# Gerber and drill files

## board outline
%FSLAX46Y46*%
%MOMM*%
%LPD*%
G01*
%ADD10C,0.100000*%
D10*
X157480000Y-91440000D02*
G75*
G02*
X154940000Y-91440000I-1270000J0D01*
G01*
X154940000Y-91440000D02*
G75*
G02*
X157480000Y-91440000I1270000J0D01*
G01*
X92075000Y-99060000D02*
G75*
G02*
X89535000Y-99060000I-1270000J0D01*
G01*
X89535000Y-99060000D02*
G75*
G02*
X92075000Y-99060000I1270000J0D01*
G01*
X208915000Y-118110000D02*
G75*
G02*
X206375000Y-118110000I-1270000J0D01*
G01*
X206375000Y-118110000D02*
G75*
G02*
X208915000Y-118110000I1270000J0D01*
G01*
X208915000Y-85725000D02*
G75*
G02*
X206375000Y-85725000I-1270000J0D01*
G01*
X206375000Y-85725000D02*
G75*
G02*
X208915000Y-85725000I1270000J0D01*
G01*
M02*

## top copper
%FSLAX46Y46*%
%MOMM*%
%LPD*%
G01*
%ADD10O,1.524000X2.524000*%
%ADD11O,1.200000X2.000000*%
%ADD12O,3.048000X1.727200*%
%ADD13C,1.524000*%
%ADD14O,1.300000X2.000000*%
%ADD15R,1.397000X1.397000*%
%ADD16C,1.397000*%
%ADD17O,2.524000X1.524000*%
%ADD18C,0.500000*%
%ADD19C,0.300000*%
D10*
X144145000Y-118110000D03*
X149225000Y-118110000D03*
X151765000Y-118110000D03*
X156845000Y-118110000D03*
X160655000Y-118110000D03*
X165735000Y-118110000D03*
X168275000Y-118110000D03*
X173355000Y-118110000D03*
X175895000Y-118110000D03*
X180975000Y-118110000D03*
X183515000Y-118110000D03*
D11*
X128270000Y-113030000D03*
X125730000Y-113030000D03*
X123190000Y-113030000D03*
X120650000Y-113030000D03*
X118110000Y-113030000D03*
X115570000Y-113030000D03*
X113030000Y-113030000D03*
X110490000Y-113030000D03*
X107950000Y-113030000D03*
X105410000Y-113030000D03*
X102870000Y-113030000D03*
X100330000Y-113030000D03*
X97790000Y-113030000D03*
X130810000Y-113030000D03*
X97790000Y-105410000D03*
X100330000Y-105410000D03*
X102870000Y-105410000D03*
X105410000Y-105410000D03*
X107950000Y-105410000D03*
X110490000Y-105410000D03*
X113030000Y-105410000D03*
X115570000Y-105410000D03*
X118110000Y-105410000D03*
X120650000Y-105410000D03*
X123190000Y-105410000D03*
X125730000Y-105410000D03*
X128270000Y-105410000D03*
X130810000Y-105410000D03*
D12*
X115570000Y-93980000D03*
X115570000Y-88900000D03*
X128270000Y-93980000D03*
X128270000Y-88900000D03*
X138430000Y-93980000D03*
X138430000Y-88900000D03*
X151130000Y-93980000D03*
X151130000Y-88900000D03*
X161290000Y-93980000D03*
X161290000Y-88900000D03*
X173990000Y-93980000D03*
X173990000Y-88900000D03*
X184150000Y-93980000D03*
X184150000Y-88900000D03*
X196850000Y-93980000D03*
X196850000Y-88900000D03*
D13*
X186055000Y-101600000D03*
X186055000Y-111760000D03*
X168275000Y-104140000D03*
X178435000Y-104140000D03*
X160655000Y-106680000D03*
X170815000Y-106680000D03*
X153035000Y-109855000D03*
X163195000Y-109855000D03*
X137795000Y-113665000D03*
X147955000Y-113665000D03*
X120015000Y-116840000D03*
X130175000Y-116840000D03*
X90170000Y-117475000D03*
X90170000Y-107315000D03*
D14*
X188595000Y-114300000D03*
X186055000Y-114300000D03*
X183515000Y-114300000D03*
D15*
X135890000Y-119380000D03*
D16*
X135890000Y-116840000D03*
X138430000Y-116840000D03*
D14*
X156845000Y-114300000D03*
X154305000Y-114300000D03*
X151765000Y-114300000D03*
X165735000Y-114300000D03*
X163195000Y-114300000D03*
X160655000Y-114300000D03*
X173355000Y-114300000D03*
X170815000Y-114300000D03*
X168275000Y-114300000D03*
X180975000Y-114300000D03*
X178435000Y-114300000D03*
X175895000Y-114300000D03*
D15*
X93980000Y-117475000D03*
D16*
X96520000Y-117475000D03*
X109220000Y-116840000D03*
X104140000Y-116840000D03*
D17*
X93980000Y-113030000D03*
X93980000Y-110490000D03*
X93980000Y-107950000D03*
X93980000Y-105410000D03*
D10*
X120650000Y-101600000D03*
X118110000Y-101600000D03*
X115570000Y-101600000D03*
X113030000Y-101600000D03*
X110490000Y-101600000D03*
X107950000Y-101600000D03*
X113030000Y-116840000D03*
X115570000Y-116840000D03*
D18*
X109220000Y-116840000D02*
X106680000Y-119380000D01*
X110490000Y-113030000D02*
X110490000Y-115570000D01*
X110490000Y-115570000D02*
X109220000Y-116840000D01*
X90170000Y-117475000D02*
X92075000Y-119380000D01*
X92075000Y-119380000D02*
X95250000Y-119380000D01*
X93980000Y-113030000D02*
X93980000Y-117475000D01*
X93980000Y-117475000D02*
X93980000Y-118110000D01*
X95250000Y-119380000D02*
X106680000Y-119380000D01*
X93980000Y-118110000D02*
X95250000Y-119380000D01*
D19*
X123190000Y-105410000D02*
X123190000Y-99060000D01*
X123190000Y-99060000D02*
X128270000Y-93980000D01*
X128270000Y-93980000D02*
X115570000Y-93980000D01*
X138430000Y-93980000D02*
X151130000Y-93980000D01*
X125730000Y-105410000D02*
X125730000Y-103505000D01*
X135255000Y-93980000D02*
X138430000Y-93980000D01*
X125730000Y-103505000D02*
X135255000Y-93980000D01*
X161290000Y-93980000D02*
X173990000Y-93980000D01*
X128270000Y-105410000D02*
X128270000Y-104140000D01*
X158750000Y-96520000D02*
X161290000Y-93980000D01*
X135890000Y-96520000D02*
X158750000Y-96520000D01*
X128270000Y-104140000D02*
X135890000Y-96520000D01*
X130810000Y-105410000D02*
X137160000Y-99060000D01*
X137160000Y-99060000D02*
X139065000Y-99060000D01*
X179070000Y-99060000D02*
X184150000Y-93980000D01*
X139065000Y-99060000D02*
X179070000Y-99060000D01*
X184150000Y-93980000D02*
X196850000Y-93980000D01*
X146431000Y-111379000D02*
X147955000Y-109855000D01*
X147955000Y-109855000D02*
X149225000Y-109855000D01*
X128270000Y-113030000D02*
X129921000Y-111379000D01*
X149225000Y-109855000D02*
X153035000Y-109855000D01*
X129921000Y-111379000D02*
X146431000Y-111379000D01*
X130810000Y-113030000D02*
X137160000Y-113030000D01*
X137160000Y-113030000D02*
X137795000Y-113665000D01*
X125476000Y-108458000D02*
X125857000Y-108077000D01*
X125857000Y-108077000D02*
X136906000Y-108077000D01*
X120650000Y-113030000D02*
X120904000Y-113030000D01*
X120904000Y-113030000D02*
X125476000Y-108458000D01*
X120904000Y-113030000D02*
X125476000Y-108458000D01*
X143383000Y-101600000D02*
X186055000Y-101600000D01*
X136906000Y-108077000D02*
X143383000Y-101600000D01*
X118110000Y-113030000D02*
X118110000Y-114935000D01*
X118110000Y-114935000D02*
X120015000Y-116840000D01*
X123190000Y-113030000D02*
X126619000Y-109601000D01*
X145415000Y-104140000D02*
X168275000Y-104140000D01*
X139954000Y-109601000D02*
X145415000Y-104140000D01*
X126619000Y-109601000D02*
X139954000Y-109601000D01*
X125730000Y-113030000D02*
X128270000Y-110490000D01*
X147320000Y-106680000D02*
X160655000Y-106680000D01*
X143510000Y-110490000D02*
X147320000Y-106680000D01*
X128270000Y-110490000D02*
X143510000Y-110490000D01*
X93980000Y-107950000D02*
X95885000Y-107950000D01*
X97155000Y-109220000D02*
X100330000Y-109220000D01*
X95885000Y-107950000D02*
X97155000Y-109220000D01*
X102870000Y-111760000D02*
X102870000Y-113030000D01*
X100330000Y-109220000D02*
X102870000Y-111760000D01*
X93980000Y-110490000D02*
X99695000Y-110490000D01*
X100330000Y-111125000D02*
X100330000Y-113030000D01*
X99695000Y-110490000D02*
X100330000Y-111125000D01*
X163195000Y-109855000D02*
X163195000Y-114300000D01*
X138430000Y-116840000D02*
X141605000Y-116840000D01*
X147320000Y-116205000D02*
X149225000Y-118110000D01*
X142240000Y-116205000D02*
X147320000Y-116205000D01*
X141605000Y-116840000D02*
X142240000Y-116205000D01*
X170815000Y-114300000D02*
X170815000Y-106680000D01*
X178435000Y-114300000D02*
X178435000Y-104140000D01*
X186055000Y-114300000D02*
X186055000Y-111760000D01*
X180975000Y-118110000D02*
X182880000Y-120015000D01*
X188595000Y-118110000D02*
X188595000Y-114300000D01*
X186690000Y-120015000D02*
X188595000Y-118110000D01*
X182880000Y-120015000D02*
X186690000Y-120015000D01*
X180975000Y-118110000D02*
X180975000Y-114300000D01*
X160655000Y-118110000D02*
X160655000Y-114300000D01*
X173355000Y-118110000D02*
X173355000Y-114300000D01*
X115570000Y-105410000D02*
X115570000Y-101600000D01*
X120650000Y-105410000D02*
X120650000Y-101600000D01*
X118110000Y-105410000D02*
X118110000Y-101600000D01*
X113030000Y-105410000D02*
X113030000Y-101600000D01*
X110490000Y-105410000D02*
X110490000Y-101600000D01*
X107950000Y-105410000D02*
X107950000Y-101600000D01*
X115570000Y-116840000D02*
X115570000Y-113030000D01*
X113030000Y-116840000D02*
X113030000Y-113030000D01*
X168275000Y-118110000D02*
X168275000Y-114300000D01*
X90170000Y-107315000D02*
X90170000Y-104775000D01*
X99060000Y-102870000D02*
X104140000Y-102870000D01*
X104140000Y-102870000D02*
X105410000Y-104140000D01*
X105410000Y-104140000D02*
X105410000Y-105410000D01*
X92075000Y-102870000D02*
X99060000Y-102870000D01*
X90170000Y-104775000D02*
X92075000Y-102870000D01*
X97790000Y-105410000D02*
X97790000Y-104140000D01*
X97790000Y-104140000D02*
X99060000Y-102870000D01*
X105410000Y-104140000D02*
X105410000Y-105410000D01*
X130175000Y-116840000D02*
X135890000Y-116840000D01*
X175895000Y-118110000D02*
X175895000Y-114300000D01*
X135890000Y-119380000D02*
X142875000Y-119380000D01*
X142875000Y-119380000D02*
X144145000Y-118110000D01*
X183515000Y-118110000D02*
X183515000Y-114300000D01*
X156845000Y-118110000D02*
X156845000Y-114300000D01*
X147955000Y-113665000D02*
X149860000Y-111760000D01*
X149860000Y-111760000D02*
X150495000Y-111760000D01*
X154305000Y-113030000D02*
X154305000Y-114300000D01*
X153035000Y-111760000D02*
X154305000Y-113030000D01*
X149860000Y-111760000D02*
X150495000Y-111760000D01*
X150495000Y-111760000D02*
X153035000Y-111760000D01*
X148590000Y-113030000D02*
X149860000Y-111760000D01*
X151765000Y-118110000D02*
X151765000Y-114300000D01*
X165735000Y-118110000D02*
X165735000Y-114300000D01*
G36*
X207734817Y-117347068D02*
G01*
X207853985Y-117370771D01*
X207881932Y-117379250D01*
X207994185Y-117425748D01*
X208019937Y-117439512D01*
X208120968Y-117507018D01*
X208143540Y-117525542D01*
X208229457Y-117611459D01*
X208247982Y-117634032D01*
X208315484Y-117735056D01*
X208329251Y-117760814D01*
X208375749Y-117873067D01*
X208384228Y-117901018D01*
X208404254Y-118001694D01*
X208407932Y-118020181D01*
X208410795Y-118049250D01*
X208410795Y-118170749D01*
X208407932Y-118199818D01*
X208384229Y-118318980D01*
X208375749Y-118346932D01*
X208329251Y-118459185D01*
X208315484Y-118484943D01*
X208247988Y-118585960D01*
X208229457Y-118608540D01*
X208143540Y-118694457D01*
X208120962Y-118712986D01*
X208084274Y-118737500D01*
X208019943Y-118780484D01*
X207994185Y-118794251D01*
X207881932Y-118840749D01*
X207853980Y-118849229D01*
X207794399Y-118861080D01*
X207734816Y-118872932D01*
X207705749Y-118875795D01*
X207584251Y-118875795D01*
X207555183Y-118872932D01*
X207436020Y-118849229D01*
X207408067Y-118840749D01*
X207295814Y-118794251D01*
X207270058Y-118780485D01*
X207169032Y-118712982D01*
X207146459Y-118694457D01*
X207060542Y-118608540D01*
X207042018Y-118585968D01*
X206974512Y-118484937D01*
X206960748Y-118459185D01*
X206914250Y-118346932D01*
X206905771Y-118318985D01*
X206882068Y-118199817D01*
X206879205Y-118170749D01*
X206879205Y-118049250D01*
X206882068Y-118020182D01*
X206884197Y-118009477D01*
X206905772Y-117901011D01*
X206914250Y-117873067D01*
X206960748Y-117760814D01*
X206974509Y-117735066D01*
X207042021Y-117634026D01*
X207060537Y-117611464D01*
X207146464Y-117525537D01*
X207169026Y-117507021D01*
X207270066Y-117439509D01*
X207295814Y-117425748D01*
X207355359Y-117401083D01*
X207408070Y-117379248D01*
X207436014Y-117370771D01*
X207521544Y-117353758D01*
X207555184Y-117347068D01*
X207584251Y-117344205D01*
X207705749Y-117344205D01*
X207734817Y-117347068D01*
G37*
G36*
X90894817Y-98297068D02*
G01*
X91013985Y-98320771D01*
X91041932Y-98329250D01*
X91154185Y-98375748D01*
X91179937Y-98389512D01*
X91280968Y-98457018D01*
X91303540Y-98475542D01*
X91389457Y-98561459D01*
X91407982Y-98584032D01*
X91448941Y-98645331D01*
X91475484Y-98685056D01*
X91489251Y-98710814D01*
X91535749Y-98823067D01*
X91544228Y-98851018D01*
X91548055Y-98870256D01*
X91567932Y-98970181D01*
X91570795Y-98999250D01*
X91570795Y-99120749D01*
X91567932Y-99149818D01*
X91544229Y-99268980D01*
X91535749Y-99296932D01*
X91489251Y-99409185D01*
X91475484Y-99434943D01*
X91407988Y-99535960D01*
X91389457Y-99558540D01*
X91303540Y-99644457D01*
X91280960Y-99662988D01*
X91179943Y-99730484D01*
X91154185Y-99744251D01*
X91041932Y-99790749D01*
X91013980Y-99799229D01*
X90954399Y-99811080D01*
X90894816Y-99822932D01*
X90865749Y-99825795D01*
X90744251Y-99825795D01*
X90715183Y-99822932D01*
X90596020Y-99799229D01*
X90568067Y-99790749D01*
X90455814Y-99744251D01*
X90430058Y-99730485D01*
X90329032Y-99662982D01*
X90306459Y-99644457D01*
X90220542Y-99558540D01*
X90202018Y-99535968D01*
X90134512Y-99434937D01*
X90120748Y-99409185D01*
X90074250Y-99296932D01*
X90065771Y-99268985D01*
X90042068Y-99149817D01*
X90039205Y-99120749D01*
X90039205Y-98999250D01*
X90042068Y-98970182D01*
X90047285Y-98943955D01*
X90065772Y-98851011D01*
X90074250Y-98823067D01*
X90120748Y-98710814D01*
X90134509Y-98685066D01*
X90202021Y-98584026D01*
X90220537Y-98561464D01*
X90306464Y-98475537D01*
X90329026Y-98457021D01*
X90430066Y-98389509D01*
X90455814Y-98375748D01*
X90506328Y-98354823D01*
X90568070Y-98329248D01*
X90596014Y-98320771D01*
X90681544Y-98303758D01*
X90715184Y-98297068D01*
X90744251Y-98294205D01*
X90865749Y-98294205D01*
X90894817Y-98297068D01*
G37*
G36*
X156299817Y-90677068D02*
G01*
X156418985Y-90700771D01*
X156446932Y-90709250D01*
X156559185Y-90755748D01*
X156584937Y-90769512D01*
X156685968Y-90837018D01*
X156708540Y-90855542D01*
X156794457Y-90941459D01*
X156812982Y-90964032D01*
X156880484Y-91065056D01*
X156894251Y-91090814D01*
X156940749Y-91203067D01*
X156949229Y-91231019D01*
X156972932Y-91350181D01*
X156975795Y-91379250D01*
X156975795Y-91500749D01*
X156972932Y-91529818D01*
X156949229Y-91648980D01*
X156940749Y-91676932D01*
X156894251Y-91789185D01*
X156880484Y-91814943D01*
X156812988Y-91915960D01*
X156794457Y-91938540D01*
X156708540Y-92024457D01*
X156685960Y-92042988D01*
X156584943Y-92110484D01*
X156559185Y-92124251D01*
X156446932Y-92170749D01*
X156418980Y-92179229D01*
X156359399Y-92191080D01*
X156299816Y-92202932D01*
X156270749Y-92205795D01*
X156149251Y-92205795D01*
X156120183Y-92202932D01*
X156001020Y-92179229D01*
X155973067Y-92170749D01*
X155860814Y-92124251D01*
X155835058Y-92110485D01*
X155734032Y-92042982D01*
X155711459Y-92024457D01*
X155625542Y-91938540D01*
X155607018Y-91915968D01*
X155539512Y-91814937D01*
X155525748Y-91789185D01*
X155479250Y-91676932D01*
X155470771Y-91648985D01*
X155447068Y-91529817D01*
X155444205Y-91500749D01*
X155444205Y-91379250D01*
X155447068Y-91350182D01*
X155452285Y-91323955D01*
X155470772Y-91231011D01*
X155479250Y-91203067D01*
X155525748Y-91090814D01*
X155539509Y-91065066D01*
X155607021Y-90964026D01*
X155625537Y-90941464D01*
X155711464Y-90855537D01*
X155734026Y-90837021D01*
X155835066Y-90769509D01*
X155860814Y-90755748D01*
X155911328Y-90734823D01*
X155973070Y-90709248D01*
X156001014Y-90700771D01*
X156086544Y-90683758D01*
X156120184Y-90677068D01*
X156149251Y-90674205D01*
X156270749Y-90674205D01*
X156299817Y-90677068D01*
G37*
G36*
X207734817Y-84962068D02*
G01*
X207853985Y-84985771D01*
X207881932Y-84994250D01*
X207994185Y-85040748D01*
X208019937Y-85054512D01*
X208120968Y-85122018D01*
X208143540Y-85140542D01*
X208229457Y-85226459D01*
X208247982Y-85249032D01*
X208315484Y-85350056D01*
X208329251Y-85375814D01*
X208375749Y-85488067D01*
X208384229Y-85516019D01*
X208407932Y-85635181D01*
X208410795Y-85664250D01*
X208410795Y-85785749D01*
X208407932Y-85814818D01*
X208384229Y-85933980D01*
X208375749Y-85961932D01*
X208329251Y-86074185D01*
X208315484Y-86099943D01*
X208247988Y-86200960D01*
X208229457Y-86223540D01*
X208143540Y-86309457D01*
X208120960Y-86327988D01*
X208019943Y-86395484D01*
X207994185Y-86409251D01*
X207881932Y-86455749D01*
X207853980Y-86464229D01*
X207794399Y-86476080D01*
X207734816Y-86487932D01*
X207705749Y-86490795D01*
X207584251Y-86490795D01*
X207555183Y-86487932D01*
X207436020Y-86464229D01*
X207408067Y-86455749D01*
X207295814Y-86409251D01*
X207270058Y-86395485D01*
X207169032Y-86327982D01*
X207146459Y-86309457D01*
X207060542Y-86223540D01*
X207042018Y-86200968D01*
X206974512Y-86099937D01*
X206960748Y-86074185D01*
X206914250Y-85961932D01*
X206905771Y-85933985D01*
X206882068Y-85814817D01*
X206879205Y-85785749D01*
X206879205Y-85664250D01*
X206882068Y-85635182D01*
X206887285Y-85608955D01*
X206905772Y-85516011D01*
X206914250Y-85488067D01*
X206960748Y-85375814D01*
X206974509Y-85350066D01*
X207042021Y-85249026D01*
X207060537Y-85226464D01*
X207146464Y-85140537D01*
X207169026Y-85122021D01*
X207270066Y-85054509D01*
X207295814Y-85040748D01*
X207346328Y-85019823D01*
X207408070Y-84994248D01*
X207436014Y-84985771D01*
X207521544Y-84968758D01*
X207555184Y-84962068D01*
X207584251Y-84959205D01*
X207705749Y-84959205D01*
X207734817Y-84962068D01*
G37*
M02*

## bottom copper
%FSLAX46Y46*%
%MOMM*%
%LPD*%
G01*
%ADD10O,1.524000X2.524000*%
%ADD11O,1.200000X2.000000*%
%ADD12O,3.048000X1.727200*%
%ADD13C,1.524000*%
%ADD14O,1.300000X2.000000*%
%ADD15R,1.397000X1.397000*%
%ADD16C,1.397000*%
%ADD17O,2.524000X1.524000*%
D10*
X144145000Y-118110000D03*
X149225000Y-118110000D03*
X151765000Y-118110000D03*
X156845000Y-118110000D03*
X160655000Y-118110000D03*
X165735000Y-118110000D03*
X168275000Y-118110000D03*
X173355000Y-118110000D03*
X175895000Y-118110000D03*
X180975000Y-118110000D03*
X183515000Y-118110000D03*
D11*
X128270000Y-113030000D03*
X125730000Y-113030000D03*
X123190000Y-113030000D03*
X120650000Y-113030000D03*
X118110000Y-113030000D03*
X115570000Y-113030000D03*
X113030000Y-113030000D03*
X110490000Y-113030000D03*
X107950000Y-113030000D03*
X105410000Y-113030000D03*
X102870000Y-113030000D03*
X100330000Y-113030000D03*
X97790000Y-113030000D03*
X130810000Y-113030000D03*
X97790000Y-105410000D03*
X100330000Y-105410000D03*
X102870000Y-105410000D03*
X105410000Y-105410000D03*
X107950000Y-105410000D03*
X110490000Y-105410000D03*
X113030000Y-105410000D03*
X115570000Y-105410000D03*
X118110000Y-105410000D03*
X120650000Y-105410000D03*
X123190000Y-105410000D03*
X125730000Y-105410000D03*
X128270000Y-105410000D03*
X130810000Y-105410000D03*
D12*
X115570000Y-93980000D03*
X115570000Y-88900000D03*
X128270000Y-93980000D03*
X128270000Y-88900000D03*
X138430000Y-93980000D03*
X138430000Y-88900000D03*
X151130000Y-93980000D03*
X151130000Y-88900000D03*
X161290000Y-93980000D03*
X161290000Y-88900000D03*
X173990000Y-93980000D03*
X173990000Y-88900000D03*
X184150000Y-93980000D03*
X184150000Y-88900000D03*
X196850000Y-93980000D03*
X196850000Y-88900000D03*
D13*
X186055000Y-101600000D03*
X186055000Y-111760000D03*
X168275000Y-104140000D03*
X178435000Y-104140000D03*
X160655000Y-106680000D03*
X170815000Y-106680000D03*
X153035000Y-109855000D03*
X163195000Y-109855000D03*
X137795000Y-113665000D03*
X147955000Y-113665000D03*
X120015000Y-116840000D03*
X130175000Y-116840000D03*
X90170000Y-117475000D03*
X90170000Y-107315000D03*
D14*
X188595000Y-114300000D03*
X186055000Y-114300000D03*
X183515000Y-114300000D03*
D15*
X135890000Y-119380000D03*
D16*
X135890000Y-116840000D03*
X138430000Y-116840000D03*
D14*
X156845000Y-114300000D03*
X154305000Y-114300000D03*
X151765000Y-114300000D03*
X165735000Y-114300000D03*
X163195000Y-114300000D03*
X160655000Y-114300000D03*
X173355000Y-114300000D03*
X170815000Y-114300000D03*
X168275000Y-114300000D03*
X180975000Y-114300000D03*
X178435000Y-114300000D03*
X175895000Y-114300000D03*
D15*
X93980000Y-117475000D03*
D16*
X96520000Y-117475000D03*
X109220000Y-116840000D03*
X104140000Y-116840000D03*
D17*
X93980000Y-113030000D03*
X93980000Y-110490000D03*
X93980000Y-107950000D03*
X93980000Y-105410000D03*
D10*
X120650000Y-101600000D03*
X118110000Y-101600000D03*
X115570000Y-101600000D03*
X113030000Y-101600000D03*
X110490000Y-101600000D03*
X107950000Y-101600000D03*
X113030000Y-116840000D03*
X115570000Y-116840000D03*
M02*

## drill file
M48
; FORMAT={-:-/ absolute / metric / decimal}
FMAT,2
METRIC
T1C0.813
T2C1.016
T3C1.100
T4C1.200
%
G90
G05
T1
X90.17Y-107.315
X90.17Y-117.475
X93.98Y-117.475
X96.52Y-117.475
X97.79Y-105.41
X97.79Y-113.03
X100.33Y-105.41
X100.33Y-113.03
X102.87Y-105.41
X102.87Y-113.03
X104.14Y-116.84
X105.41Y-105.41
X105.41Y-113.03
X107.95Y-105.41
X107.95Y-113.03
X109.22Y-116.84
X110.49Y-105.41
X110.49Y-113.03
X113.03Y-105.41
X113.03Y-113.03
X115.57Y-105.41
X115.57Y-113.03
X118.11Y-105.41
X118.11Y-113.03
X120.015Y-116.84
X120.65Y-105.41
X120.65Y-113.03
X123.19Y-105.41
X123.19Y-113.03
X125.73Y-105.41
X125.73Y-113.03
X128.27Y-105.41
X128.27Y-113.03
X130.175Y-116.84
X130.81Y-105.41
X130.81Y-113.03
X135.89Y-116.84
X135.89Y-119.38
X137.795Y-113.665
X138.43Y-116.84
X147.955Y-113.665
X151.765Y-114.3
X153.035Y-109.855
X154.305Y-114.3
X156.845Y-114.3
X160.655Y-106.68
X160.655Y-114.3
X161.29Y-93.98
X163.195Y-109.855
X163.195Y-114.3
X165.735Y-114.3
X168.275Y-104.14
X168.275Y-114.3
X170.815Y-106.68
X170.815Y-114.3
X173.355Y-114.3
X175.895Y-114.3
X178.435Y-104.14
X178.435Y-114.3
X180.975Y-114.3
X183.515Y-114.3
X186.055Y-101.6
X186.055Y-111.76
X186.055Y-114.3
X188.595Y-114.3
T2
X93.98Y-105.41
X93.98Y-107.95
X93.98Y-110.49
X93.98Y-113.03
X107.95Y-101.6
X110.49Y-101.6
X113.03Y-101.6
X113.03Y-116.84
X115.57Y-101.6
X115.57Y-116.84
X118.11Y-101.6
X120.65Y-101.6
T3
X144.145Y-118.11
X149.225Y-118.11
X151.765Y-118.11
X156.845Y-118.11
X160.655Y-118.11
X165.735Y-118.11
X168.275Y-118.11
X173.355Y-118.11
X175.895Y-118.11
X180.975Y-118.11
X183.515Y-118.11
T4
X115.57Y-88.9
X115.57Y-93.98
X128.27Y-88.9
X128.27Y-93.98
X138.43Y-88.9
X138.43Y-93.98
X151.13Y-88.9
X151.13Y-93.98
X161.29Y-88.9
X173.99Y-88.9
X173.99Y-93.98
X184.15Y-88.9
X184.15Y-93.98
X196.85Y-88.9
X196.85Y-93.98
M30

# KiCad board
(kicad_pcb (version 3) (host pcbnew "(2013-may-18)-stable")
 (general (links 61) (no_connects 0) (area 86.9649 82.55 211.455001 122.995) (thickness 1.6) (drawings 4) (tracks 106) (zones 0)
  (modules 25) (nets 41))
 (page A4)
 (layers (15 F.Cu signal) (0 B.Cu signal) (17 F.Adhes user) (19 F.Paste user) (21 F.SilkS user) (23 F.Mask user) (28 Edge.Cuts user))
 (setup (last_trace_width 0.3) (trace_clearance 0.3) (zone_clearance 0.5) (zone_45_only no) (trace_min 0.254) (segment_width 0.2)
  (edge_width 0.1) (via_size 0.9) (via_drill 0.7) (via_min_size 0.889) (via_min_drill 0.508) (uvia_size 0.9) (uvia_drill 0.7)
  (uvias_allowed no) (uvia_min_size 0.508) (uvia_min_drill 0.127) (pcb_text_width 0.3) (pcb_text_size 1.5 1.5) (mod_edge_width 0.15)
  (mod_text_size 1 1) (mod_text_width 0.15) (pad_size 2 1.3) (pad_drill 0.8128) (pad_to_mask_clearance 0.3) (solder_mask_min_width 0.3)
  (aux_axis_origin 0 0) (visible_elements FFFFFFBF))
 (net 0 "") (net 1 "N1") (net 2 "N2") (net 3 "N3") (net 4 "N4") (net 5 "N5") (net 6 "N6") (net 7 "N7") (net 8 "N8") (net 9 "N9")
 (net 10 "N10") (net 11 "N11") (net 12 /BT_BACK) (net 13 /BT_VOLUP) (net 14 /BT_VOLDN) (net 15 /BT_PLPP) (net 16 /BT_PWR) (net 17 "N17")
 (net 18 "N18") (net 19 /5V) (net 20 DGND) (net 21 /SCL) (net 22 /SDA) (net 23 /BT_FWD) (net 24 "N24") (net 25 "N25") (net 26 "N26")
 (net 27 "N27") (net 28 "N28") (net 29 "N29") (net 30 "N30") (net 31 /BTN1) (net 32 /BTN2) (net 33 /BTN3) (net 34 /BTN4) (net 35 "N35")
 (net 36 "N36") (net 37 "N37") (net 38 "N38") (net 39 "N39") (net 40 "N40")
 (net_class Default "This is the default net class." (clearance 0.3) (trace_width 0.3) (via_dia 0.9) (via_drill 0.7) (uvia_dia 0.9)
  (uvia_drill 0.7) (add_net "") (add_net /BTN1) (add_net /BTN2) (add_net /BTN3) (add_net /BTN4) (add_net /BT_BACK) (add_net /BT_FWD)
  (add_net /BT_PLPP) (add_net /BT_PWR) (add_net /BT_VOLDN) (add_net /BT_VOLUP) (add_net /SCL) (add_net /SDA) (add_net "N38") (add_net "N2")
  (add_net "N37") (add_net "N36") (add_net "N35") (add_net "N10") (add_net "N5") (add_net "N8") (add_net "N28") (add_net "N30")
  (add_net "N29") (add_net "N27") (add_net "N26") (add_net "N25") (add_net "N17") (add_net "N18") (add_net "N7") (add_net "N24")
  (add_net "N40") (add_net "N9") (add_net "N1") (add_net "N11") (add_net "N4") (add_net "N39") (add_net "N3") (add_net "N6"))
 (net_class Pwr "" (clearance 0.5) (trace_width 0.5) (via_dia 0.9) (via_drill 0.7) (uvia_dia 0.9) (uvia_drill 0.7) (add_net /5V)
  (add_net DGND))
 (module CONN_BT (layer F.Cu) (at 160.655 118.11)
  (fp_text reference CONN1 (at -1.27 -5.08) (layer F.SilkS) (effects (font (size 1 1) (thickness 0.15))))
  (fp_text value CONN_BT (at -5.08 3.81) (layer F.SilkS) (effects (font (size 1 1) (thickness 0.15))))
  (pad pwr1 thru_hole oval (at -16.51 0) (size 1.524 2.524) (drill 1.1) (layers *.Cu *.Mask) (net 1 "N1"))
  (pad pwr2 thru_hole oval (at -11.43 0) (size 1.524 2.524) (drill 1.1) (layers *.Cu *.Mask) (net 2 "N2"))
  (pad fwd thru_hole oval (at -8.89 0) (size 1.524 2.524) (drill 1.1) (layers *.Cu *.Mask) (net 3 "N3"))
  (pad 1V81 thru_hole oval (at -3.81 0) (size 1.524 2.524) (drill 1.1) (layers *.Cu *.Mask) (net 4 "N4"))
  (pad back thru_hole oval (at 0 0) (size 1.524 2.524) (drill 1.1) (layers *.Cu *.Mask) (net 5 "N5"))
  (pad 1V82 thru_hole oval (at 5.08 0) (size 1.524 2.524) (drill 1.1) (layers *.Cu *.Mask) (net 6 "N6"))
  (pad v_up thru_hole oval (at 7.62 0) (size 1.524 2.524) (drill 1.1) (layers *.Cu *.Mask) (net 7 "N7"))
  (pad 1V83 thru_hole oval (at 12.7 0) (size 1.524 2.524) (drill 1.1) (layers *.Cu *.Mask) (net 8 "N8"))
  (pad v_dn thru_hole oval (at 15.24 0) (size 1.524 2.524) (drill 1.1) (layers *.Cu *.Mask) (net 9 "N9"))
  (pad 1V84 thru_hole oval (at 20.32 0) (size 1.524 2.524) (drill 1.1) (layers *.Cu *.Mask) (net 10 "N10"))
  (pad play thru_hole oval (at 22.86 0) (size 1.524 2.524) (drill 1.1) (layers *.Cu *.Mask) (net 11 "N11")))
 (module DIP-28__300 (layer B.Cu) (at 114.3 109.22 180)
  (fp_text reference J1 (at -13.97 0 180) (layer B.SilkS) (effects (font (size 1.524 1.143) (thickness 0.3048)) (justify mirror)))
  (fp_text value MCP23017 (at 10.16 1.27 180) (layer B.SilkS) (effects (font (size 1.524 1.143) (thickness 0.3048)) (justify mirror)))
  (pad 2 thru_hole oval (at -13.97 -3.81 180) (size 1.2 2) (drill 0.8128) (layers *.Cu *.Mask) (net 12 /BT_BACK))
  (pad 3 thru_hole oval (at -11.43 -3.81 180) (size 1.2 2) (drill 0.8128) (layers *.Cu *.Mask) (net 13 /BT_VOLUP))
  (pad 4 thru_hole oval (at -8.89 -3.81 180) (size 1.2 2) (drill 0.8128) (layers *.Cu *.Mask) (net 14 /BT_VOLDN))
  (pad 5 thru_hole oval (at -6.35 -3.81 180) (size 1.2 2) (drill 0.8128) (layers *.Cu *.Mask) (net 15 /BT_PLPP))
  (pad 6 thru_hole oval (at -3.81 -3.81 180) (size 1.2 2) (drill 0.8128) (layers *.Cu *.Mask) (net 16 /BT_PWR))
  (pad 7 thru_hole oval (at -1.27 -3.81 180) (size 1.2 2) (drill 0.8128) (layers *.Cu *.Mask) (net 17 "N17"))
  (pad 8 thru_hole oval (at 1.27 -3.81 180) (size 1.2 2) (drill 0.8128) (layers *.Cu *.Mask) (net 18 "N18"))
  (pad 9 thru_hole oval (at 3.81 -3.81 180) (size 1.2 2) (drill 0.8128) (layers *.Cu *.Mask) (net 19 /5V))
  (pad 10 thru_hole oval (at 6.35 -3.81 180) (size 1.2 2) (drill 0.8128) (layers *.Cu *.Mask) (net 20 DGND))
  (pad 11 thru_hole oval (at 8.89 -3.81 180) (size 1.2 2) (drill 0.8128) (layers *.Cu *.Mask))
  (pad 12 thru_hole oval (at 11.43 -3.81 180) (size 1.2 2) (drill 0.8128) (layers *.Cu *.Mask) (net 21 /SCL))
  (pad 13 thru_hole oval (at 13.97 -3.81 180) (size 1.2 2) (drill 0.8128) (layers *.Cu *.Mask) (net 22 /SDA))
  (pad 14 thru_hole oval (at 16.51 -3.81 180) (size 1.2 2) (drill 0.8128) (layers *.Cu *.Mask))
  (pad 1 thru_hole oval (at -16.51 -3.81 180) (size 1.2 2) (drill 0.8128) (layers *.Cu *.Mask) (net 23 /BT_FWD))
  (pad 15 thru_hole oval (at 16.51 3.81 180) (size 1.2 2) (drill 0.8128) (layers *.Cu *.Mask) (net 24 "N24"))
  (pad 16 thru_hole oval (at 13.97 3.81 180) (size 1.2 2) (drill 0.8128) (layers *.Cu *.Mask) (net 20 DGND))
  (pad 17 thru_hole oval (at 11.43 3.81 180) (size 1.2 2) (drill 0.8128) (layers *.Cu *.Mask) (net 20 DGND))
  (pad 18 thru_hole oval (at 8.89 3.81 180) (size 1.2 2) (drill 0.8128) (layers *.Cu *.Mask) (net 24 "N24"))
  (pad 19 thru_hole oval (at 6.35 3.81 180) (size 1.2 2) (drill 0.8128) (layers *.Cu *.Mask) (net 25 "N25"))
  (pad 20 thru_hole oval (at 3.81 3.81 180) (size 1.2 2) (drill 0.8128) (layers *.Cu *.Mask) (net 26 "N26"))
  (pad 21 thru_hole oval (at 1.27 3.81 180) (size 1.2 2) (drill 0.8128) (layers *.Cu *.Mask) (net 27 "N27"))
  (pad 22 thru_hole oval (at -1.27 3.81 180) (size 1.2 2) (drill 0.8128) (layers *.Cu *.Mask) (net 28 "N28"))
  (pad 23 thru_hole oval (at -3.81 3.81 180) (size 1.2 2) (drill 0.8128) (layers *.Cu *.Mask) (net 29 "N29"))
  (pad 24 thru_hole oval (at -6.35 3.81 180) (size 1.2 2) (drill 0.8128) (layers *.Cu *.Mask) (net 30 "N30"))
  (pad 25 thru_hole oval (at -8.89 3.81 180) (size 1.2 2) (drill 0.8128) (layers *.Cu *.Mask) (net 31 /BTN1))
  (pad 26 thru_hole oval (at -11.43 3.81 180) (size 1.2 2) (drill 0.8128) (layers *.Cu *.Mask) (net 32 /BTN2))
  (pad 27 thru_hole oval (at -13.97 3.81 180) (size 1.2 2) (drill 0.8128) (layers *.Cu *.Mask) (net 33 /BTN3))
  (pad 28 thru_hole oval (at -16.51 3.81 180) (size 1.2 2) (drill 0.8128) (layers *.Cu *.Mask) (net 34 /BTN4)))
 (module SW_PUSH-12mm (layer F.Cu) (at 121.92 91.44 180)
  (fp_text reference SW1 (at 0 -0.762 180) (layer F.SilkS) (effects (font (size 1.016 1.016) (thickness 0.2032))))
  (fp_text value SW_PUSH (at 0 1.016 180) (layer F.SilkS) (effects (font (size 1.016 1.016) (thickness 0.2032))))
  (pad 1 thru_hole oval (at 6.35 -2.54 180) (size 3.048 1.7272) (drill 1.2) (layers *.Cu *.Mask F.SilkS) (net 31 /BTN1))
  (pad 2 thru_hole oval (at 6.35 2.54 180) (size 3.048 1.7272) (drill 1.2) (layers *.Cu *.Mask F.SilkS) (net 20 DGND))
  (pad 1 thru_hole oval (at -6.35 -2.54 180) (size 3.048 1.7272) (drill 1.2) (layers *.Cu *.Mask F.SilkS) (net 31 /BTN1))
  (pad 2 thru_hole oval (at -6.35 2.54 180) (size 3.048 1.7272) (drill 1.2) (layers *.Cu *.Mask F.SilkS) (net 20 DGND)))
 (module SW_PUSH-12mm (layer F.Cu) (at 144.78 91.44 180)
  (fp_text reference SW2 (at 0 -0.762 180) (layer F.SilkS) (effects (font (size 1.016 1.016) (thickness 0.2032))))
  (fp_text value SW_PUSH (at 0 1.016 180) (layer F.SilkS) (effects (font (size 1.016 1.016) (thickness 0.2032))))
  (pad 1 thru_hole oval (at 6.35 -2.54 180) (size 3.048 1.7272) (drill 1.2) (layers *.Cu *.Mask F.SilkS) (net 32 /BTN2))
  (pad 2 thru_hole oval (at 6.35 2.54 180) (size 3.048 1.7272) (drill 1.2) (layers *.Cu *.Mask F.SilkS) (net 20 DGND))
  (pad 1 thru_hole oval (at -6.35 -2.54 180) (size 3.048 1.7272) (drill 1.2) (layers *.Cu *.Mask F.SilkS) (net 32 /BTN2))
  (pad 2 thru_hole oval (at -6.35 2.54 180) (size 3.048 1.7272) (drill 1.2) (layers *.Cu *.Mask F.SilkS) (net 20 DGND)))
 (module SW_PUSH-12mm (layer F.Cu) (at 167.64 91.44 180)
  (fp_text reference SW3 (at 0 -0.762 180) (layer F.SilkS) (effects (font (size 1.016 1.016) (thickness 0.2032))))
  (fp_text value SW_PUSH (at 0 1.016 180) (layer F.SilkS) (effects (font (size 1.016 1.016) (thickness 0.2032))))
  (pad 1 thru_hole oval (at 6.35 -2.54 180) (size 3.048 1.7272) (drill 0.8128) (layers *.Cu *.Mask F.SilkS) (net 33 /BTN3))
  (pad 2 thru_hole oval (at 6.35 2.54 180) (size 3.048 1.7272) (drill 1.2) (layers *.Cu *.Mask F.SilkS) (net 20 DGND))
  (pad 1 thru_hole oval (at -6.35 -2.54 180) (size 3.048 1.7272) (drill 1.2) (layers *.Cu *.Mask F.SilkS) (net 33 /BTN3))
  (pad 2 thru_hole oval (at -6.35 2.54 180) (size 3.048 1.7272) (drill 1.2) (layers *.Cu *.Mask F.SilkS) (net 20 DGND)))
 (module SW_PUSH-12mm (layer F.Cu) (at 190.5 91.44 180)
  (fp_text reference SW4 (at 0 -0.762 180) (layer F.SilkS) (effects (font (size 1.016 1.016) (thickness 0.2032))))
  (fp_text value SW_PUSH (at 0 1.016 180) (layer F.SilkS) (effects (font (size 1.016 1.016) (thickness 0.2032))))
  (pad 1 thru_hole oval (at 6.35 -2.54 180) (size 3.048 1.7272) (drill 1.2) (layers *.Cu *.Mask F.SilkS) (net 34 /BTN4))
  (pad 2 thru_hole oval (at 6.35 2.54 180) (size 3.048 1.7272) (drill 1.2) (layers *.Cu *.Mask F.SilkS) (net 20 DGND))
  (pad 1 thru_hole oval (at -6.35 -2.54 180) (size 3.048 1.7272) (drill 1.2) (layers *.Cu *.Mask F.SilkS) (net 34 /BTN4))
  (pad 2 thru_hole oval (at -6.35 2.54 180) (size 3.048 1.7272) (drill 1.2) (layers *.Cu *.Mask F.SilkS) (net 20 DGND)))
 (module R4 (layer B.Cu) (at 186.055 106.68 270) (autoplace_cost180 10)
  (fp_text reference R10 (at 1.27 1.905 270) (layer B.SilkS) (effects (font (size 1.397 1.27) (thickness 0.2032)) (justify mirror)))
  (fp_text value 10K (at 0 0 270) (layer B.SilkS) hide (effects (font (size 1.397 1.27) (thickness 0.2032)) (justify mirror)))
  (pad 1 thru_hole circle (at -5.08 0 270) (size 1.524 1.524) (drill 0.8128) (layers *.Cu *.Mask) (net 15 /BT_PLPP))
  (pad 2 thru_hole circle (at 5.08 0 270) (size 1.524 1.524) (drill 0.8128) (layers *.Cu *.Mask) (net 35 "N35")))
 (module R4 (layer B.Cu) (at 173.355 104.14) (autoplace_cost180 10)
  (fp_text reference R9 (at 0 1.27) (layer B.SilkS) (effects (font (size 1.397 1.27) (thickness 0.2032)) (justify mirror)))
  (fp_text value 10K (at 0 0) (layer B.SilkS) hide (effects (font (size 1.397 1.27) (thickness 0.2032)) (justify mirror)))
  (pad 1 thru_hole circle (at -5.08 0) (size 1.524 1.524) (drill 0.8128) (layers *.Cu *.Mask) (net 14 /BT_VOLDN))
  (pad 2 thru_hole circle (at 5.08 0) (size 1.524 1.524) (drill 0.8128) (layers *.Cu *.Mask) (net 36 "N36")))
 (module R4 (layer B.Cu) (at 165.735 106.68) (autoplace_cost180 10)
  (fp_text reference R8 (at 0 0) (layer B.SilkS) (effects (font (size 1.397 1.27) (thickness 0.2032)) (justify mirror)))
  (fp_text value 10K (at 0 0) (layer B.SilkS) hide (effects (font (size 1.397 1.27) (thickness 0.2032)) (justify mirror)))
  (pad 1 thru_hole circle (at -5.08 0) (size 1.524 1.524) (drill 0.8128) (layers *.Cu *.Mask) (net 13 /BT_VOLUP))
  (pad 2 thru_hole circle (at 5.08 0) (size 1.524 1.524) (drill 0.8128) (layers *.Cu *.Mask) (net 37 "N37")))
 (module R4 (layer B.Cu) (at 158.115 109.855) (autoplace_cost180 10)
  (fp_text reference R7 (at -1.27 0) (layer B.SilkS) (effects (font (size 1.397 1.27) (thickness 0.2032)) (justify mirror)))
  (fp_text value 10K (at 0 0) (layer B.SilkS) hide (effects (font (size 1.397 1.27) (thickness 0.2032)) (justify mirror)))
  (pad 1 thru_hole circle (at -5.08 0) (size 1.524 1.524) (drill 0.8128) (layers *.Cu *.Mask) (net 12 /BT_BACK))
  (pad 2 thru_hole circle (at 5.08 0) (size 1.524 1.524) (drill 0.8128) (layers *.Cu *.Mask) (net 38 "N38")))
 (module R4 (layer B.Cu) (at 142.875 113.665) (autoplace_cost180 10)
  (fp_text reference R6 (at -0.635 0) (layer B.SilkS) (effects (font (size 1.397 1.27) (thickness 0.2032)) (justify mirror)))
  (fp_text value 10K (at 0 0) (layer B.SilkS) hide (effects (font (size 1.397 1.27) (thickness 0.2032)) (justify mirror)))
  (pad 1 thru_hole circle (at -5.08 0) (size 1.524 1.524) (drill 0.8128) (layers *.Cu *.Mask) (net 23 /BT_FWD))
  (pad 2 thru_hole circle (at 5.08 0) (size 1.524 1.524) (drill 0.8128) (layers *.Cu *.Mask) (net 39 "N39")))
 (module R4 (layer B.Cu) (at 125.095 116.84) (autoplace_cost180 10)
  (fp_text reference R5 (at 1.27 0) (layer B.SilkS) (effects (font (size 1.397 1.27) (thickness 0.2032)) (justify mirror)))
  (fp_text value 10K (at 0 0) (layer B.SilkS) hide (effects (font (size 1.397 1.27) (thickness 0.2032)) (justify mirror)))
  (pad 1 thru_hole circle (at -5.08 0) (size 1.524 1.524) (drill 0.8128) (layers *.Cu *.Mask) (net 16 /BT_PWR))
  (pad 2 thru_hole circle (at 5.08 0) (size 1.524 1.524) (drill 0.8128) (layers *.Cu *.Mask) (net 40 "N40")))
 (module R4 (layer B.Cu) (at 90.17 112.395 90) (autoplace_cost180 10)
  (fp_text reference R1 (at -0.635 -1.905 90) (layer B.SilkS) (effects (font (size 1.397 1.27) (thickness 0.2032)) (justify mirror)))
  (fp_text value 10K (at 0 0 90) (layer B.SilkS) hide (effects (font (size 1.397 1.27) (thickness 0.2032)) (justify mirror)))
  (pad 1 thru_hole circle (at -5.08 0 90) (size 1.524 1.524) (drill 0.8128) (layers *.Cu *.Mask) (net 19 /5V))
  (pad 2 thru_hole circle (at 5.08 0 90) (size 1.524 1.524) (drill 0.8128) (layers *.Cu *.Mask) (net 24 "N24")))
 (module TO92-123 (layer B.Cu) (at 184.785 113.03 90)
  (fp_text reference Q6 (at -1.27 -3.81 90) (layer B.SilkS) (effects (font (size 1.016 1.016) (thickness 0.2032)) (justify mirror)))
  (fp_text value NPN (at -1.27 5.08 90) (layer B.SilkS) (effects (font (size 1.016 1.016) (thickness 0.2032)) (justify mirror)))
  (pad 3 thru_hole oval (at -1.27 3.81 90) (size 2 1.3) (drill 0.8128) (layers *.Cu *.Mask) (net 10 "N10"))
  (pad 2 thru_hole oval (at -1.27 1.27 90) (size 2 1.3) (drill 0.8128) (layers *.Cu *.Mask) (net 35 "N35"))
  (pad 1 thru_hole oval (at -1.27 -1.27 90) (size 2 1.3) (drill 0.8128) (layers *.Cu *.Mask) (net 11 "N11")))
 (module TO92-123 (layer B.Cu) (at 137.16 118.11 270)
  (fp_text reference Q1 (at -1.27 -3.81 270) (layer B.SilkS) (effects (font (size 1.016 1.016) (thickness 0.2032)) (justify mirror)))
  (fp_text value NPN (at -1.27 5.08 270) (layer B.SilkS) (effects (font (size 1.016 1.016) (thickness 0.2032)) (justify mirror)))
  (pad 3 thru_hole rect (at 1.27 1.27 270) (size 1.397 1.397) (drill 0.8128) (layers *.Cu *.Mask) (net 1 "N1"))
  (pad 2 thru_hole circle (at -1.27 1.27 270) (size 1.397 1.397) (drill 0.8128) (layers *.Cu *.Mask) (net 40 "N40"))
  (pad 1 thru_hole circle (at -1.27 -1.27 270) (size 1.397 1.397) (drill 0.8128) (layers *.Cu *.Mask) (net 2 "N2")))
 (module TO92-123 (layer B.Cu) (at 153.035 113.03 90)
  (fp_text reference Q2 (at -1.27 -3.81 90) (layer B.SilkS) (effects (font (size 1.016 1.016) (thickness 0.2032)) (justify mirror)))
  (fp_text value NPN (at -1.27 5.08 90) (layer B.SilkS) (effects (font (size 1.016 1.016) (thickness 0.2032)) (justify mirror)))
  (pad 3 thru_hole oval (at -1.27 3.81 90) (size 2 1.3) (drill 0.8128) (layers *.Cu *.Mask) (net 4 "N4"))
  (pad 2 thru_hole oval (at -1.27 1.27 90) (size 2 1.3) (drill 0.8128) (layers *.Cu *.Mask) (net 39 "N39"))
  (pad 1 thru_hole oval (at -1.27 -1.27 90) (size 2 1.3) (drill 0.8128) (layers *.Cu *.Mask) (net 3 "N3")))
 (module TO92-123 (layer B.Cu) (at 161.925 113.03 90)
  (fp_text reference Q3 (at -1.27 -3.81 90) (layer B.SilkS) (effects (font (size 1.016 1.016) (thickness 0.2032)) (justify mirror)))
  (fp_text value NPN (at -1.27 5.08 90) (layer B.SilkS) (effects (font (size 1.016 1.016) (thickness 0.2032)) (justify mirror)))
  (pad 3 thru_hole oval (at -1.27 3.81 90) (size 2 1.3) (drill 0.8128) (layers *.Cu *.Mask) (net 6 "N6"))
  (pad 2 thru_hole oval (at -1.27 1.27 90) (size 2 1.3) (drill 0.8128) (layers *.Cu *.Mask) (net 38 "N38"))
  (pad 1 thru_hole oval (at -1.27 -1.27 90) (size 2 1.3) (drill 0.8128) (layers *.Cu *.Mask) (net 5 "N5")))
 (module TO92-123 (layer B.Cu) (at 169.545 113.03 90)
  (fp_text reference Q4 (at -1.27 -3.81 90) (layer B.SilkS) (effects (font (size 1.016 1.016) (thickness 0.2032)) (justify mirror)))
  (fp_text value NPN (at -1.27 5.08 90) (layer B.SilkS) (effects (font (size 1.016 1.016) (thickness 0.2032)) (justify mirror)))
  (pad 3 thru_hole oval (at -1.27 3.81 90) (size 2 1.3) (drill 0.8128) (layers *.Cu *.Mask) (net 8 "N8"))
  (pad 2 thru_hole oval (at -1.27 1.27 90) (size 2 1.3) (drill 0.8128) (layers *.Cu *.Mask) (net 37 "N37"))
  (pad 1 thru_hole oval (at -1.27 -1.27 90) (size 2 1.3) (drill 0.8128) (layers *.Cu *.Mask) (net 7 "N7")))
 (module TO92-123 (layer B.Cu) (at 177.165 113.03 90)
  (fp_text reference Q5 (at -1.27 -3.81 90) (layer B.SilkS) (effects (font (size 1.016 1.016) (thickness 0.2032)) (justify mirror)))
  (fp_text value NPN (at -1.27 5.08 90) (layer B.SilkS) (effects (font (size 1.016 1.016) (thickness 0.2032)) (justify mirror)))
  (pad 3 thru_hole oval (at -1.27 3.81 90) (size 2 1.3) (drill 0.8128) (layers *.Cu *.Mask) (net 10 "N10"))
  (pad 2 thru_hole oval (at -1.27 1.27 90) (size 2 1.3) (drill 0.8128) (layers *.Cu *.Mask) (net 36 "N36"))
  (pad 1 thru_hole oval (at -1.27 -1.27 90) (size 2 1.3) (drill 0.8128) (layers *.Cu *.Mask) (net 9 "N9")))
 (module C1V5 (layer B.Cu) (at 95.25 117.475)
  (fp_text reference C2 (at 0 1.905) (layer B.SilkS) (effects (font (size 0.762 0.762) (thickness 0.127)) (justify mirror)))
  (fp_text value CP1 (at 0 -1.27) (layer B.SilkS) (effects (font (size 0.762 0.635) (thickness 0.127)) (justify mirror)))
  (pad 1 thru_hole rect (at -1.27 0) (size 1.397 1.397) (drill 0.8128) (layers *.Cu *.Mask) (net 19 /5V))
  (pad 2 thru_hole circle (at 1.27 0) (size 1.397 1.397) (drill 0.8128) (layers *.Cu *.Mask) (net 20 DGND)))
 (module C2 (layer B.Cu) (at 106.68 116.84 180)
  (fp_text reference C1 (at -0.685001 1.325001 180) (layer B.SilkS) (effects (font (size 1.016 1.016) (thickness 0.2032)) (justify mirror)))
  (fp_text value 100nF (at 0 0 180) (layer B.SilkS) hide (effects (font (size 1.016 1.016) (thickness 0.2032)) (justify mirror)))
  (pad 1 thru_hole circle (at -2.54 0 180) (size 1.397 1.397) (drill 0.8128) (layers *.Cu *.Mask) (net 19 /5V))
  (pad 2 thru_hole circle (at 2.54 0 180) (size 1.397 1.397) (drill 0.8128) (layers *.Cu *.Mask) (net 20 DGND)))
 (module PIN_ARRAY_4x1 (layer B.Cu) (at 93.98 109.22 90)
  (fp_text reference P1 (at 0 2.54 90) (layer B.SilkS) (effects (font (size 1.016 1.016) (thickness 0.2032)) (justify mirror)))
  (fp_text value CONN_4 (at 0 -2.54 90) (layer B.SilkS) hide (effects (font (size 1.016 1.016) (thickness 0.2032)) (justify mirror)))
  (pad 1 thru_hole oval (at -3.81 0 90) (size 1.524 2.524) (drill 1.016) (layers *.Cu *.Mask) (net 19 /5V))
  (pad 2 thru_hole oval (at -1.27 0 90) (size 1.524 2.524) (drill 1.016) (layers *.Cu *.Mask) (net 22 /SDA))
  (pad 3 thru_hole oval (at 1.27 0 90) (size 1.524 2.524) (drill 1.016) (layers *.Cu *.Mask) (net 21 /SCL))
  (pad 4 thru_hole oval (at 3.81 0 90) (size 1.524 2.524) (drill 1.016) (layers *.Cu *.Mask) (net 20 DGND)))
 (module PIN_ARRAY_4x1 (layer B.Cu) (at 116.84 101.6 180)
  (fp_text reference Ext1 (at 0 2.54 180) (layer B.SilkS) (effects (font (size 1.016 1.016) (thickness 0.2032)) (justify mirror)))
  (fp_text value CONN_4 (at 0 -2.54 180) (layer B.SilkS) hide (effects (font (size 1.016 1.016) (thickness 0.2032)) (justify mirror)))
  (pad 1 thru_hole oval (at -3.81 0 180) (size 1.524 2.524) (drill 1.016) (layers *.Cu *.Mask) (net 30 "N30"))
  (pad 2 thru_hole oval (at -1.27 0 180) (size 1.524 2.524) (drill 1.016) (layers *.Cu *.Mask) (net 29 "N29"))
  (pad 3 thru_hole oval (at 1.27 0 180) (size 1.524 2.524) (drill 1.016) (layers *.Cu *.Mask) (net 28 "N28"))
  (pad 4 thru_hole oval (at 3.81 0 180) (size 1.524 2.524) (drill 1.016) (layers *.Cu *.Mask) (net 27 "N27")))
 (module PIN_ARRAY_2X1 (layer B.Cu) (at 109.22 101.6 180)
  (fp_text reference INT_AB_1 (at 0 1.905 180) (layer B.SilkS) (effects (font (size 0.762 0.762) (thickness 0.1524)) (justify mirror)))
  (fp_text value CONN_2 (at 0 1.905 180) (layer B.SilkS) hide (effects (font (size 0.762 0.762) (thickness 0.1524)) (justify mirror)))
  (pad 1 thru_hole oval (at -1.27 0 180) (size 1.524 2.524) (drill 1.016) (layers *.Cu *.Mask) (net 26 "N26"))
  (pad 2 thru_hole oval (at 1.27 0 180) (size 1.524 2.524) (drill 1.016) (layers *.Cu *.Mask) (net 25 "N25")))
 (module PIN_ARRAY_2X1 (layer B.Cu) (at 114.3 116.84)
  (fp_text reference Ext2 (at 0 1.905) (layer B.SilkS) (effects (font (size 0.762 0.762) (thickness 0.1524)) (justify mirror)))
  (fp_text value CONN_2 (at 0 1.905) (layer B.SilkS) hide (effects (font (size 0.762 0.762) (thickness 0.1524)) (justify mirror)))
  (pad 1 thru_hole oval (at -1.27 0) (size 1.524 2.524) (drill 1.016) (layers *.Cu *.Mask) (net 18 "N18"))
  (pad 2 thru_hole oval (at 1.27 0) (size 1.524 2.524) (drill 1.016) (layers *.Cu *.Mask) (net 17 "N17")))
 (gr_circle (center 156.21 91.44) (end 157.48 91.44) (layer Edge.Cuts) (width 0.1))
 (gr_circle (center 90.805 99.06) (end 92.075 99.06) (layer Edge.Cuts) (width 0.1))
 (gr_circle (center 207.645 118.11) (end 206.375 118.11) (layer Edge.Cuts) (width 0.1))
 (gr_circle (center 207.645 85.725) (end 206.375 85.725) (layer Edge.Cuts) (width 0.1))
 (segment (start 109.22 116.84) (end 106.68 119.38) (width 0.5) (layer F.Cu) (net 19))
 (segment (start 110.49 113.03) (end 110.49 115.57) (width 0.5) (layer F.Cu) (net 19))
 (segment (start 110.49 115.57) (end 109.22 116.84) (width 0.5) (layer F.Cu) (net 19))
 (segment (start 90.17 117.475) (end 92.075 119.38) (width 0.5) (layer F.Cu) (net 19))
 (segment (start 92.075 119.38) (end 95.25 119.38) (width 0.5) (layer F.Cu) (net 19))
 (segment (start 93.98 113.03) (end 93.98 117.475) (width 0.5) (layer F.Cu) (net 19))
 (segment (start 93.98 117.475) (end 93.98 118.11) (width 0.5) (layer F.Cu) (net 19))
 (segment (start 95.25 119.38) (end 106.68 119.38) (width 0.5) (layer F.Cu) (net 19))
 (segment (start 93.98 118.11) (end 95.25 119.38) (width 0.5) (layer F.Cu) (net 19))
 (segment (start 123.19 105.41) (end 123.19 99.06) (width 0.3) (layer F.Cu) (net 31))
 (segment (start 123.19 99.06) (end 128.27 93.98) (width 0.3) (layer F.Cu) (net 31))
 (segment (start 128.27 93.98) (end 115.57 93.98) (width 0.3) (layer F.Cu) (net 31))
 (segment (start 138.43 93.98) (end 151.13 93.98) (width 0.3) (layer F.Cu) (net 32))
 (segment (start 125.73 105.41) (end 125.73 103.505) (width 0.3) (layer F.Cu) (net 32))
 (segment (start 135.255 93.98) (end 138.43 93.98) (width 0.3) (layer F.Cu) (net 32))
 (segment (start 125.73 103.505) (end 135.255 93.98) (width 0.3) (layer F.Cu) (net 32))
 (segment (start 161.29 93.98) (end 173.99 93.98) (width 0.3) (layer F.Cu) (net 33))
 (segment (start 128.27 105.41) (end 128.27 104.14) (width 0.3) (layer F.Cu) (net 33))
 (segment (start 158.75 96.52) (end 161.29 93.98) (width 0.3) (layer F.Cu) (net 33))
 (segment (start 135.89 96.52) (end 158.75 96.52) (width 0.3) (layer F.Cu) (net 33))
 (segment (start 128.27 104.14) (end 135.89 96.52) (width 0.3) (layer F.Cu) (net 33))
 (segment (start 130.81 105.41) (end 137.16 99.06) (width 0.3) (layer F.Cu) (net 34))
 (segment (start 137.16 99.06) (end 139.065 99.06) (width 0.3) (layer F.Cu) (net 34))
 (segment (start 179.07 99.06) (end 184.15 93.98) (width 0.3) (layer F.Cu) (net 34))
 (segment (start 139.065 99.06) (end 179.07 99.06) (width 0.3) (layer F.Cu) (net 34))
 (segment (start 184.15 93.98) (end 196.85 93.98) (width 0.3) (layer F.Cu) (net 34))
 (segment (start 146.431 111.379) (end 147.955 109.855) (width 0.3) (layer F.Cu) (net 12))
 (segment (start 147.955 109.855) (end 149.225 109.855) (width 0.3) (layer F.Cu) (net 12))
 (segment (start 128.27 113.03) (end 129.921 111.379) (width 0.3) (layer F.Cu) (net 12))
 (segment (start 149.225 109.855) (end 153.035 109.855) (width 0.3) (layer F.Cu) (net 12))
 (segment (start 129.921 111.379) (end 146.431 111.379) (width 0.3) (layer F.Cu) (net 12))
 (segment (start 130.81 113.03) (end 137.16 113.03) (width 0.3) (layer F.Cu) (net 23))
 (segment (start 137.16 113.03) (end 137.795 113.665) (width 0.3) (layer F.Cu) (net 23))
 (segment (start 125.476 108.458) (end 125.857 108.077) (width 0.3) (layer F.Cu) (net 15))
 (segment (start 125.857 108.077) (end 136.906 108.077) (width 0.3) (layer F.Cu) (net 15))
 (segment (start 120.65 113.03) (end 120.904 113.03) (width 0.3) (layer F.Cu) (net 15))
 (segment (start 120.904 113.03) (end 125.476 108.458) (width 0.3) (layer F.Cu) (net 15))
 (segment (start 120.904 113.03) (end 125.476 108.458) (width 0.3) (layer F.Cu) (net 15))
 (segment (start 143.383 101.6) (end 186.055 101.6) (width 0.3) (layer F.Cu) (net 15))
 (segment (start 136.906 108.077) (end 143.383 101.6) (width 0.3) (layer F.Cu) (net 15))
 (segment (start 118.11 113.03) (end 118.11 114.935) (width 0.3) (layer F.Cu) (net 16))
 (segment (start 118.11 114.935) (end 120.015 116.84) (width 0.3) (layer F.Cu) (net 16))
 (segment (start 123.19 113.03) (end 126.619 109.601) (width 0.3) (layer F.Cu) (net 14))
 (segment (start 145.415 104.14) (end 168.275 104.14) (width 0.3) (layer F.Cu) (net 14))
 (segment (start 139.954 109.601) (end 145.415 104.14) (width 0.3) (layer F.Cu) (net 14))
 (segment (start 126.619 109.601) (end 139.954 109.601) (width 0.3) (layer F.Cu) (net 14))
 (segment (start 125.73 113.03) (end 128.27 110.49) (width 0.3) (layer F.Cu) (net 13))
 (segment (start 147.32 106.68) (end 160.655 106.68) (width 0.3) (layer F.Cu) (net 13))
 (segment (start 143.51 110.49) (end 147.32 106.68) (width 0.3) (layer F.Cu) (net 13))
 (segment (start 128.27 110.49) (end 143.51 110.49) (width 0.3) (layer F.Cu) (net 13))
 (segment (start 93.98 107.95) (end 95.885 107.95) (width 0.3) (layer F.Cu) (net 21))
 (segment (start 97.155 109.22) (end 100.33 109.22) (width 0.3) (layer F.Cu) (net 21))
 (segment (start 95.885 107.95) (end 97.155 109.22) (width 0.3) (layer F.Cu) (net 21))
 (segment (start 102.87 111.76) (end 102.87 113.03) (width 0.3) (layer F.Cu) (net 21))
 (segment (start 100.33 109.22) (end 102.87 111.76) (width 0.3) (layer F.Cu) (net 21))
 (segment (start 93.98 110.49) (end 99.695 110.49) (width 0.3) (layer F.Cu) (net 22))
 (segment (start 100.33 111.125) (end 100.33 113.03) (width 0.3) (layer F.Cu) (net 22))
 (segment (start 99.695 110.49) (end 100.33 111.125) (width 0.3) (layer F.Cu) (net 22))
 (segment (start 163.195 109.855) (end 163.195 114.3) (width 0.3) (layer F.Cu) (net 38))
 (segment (start 138.43 116.84) (end 141.605 116.84) (width 0.3) (layer F.Cu) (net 2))
 (segment (start 147.32 116.205) (end 149.225 118.11) (width 0.3) (layer F.Cu) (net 2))
 (segment (start 142.24 116.205) (end 147.32 116.205) (width 0.3) (layer F.Cu) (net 2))
 (segment (start 141.605 116.84) (end 142.24 116.205) (width 0.3) (layer F.Cu) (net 2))
 (segment (start 170.815 114.3) (end 170.815 106.68) (width 0.3) (layer F.Cu) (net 37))
 (segment (start 178.435 114.3) (end 178.435 104.14) (width 0.3) (layer F.Cu) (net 36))
 (segment (start 186.055 114.3) (end 186.055 111.76) (width 0.3) (layer F.Cu) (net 35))
 (segment (start 180.975 118.11) (end 182.88 120.015) (width 0.3) (layer F.Cu) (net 10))
 (segment (start 188.595 118.11) (end 188.595 114.3) (width 0.3) (layer F.Cu) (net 10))
 (segment (start 186.69 120.015) (end 188.595 118.11) (width 0.3) (layer F.Cu) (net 10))
 (segment (start 182.88 120.015) (end 186.69 120.015) (width 0.3) (layer F.Cu) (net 10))
 (segment (start 180.975 118.11) (end 180.975 114.3) (width 0.3) (layer F.Cu) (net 10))
 (segment (start 160.655 118.11) (end 160.655 114.3) (width 0.3) (layer F.Cu) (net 5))
 (segment (start 173.355 118.11) (end 173.355 114.3) (width 0.3) (layer F.Cu) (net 8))
 (segment (start 115.57 105.41) (end 115.57 101.6) (width 0.3) (layer F.Cu) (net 28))
 (segment (start 120.65 105.41) (end 120.65 101.6) (width 0.3) (layer F.Cu) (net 30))
 (segment (start 118.11 105.41) (end 118.11 101.6) (width 0.3) (layer F.Cu) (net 29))
 (segment (start 113.03 105.41) (end 113.03 101.6) (width 0.3) (layer F.Cu) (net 27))
 (segment (start 110.49 105.41) (end 110.49 101.6) (width 0.3) (layer F.Cu) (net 26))
 (segment (start 107.95 105.41) (end 107.95 101.6) (width 0.3) (layer F.Cu) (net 25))
 (segment (start 115.57 116.84) (end 115.57 113.03) (width 0.3) (layer F.Cu) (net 17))
 (segment (start 113.03 116.84) (end 113.03 113.03) (width 0.3) (layer F.Cu) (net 18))
 (segment (start 168.275 118.11) (end 168.275 114.3) (width 0.3) (layer F.Cu) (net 7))
 (segment (start 90.17 107.315) (end 90.17 104.775) (width 0.3) (layer F.Cu) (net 24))
 (segment (start 99.06 102.87) (end 104.14 102.87) (width 0.3) (layer F.Cu) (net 24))
 (segment (start 104.14 102.87) (end 105.41 104.14) (width 0.3) (layer F.Cu) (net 24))
 (segment (start 105.41 104.14) (end 105.41 105.41) (width 0.3) (layer F.Cu) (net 24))
 (segment (start 92.075 102.87) (end 99.06 102.87) (width 0.3) (layer F.Cu) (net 24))
 (segment (start 90.17 104.775) (end 92.075 102.87) (width 0.3) (layer F.Cu) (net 24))
 (segment (start 97.79 105.41) (end 97.79 104.14) (width 0.3) (layer F.Cu) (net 24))
 (segment (start 97.79 104.14) (end 99.06 102.87) (width 0.3) (layer F.Cu) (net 24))
 (segment (start 105.41 104.14) (end 105.41 105.41) (width 0.3) (layer F.Cu) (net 24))
 (segment (start 130.175 116.84) (end 135.89 116.84) (width 0.3) (layer F.Cu) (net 40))
 (segment (start 175.895 118.11) (end 175.895 114.3) (width 0.3) (layer F.Cu) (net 9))
 (segment (start 135.89 119.38) (end 142.875 119.38) (width 0.3) (layer F.Cu) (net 1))
 (segment (start 142.875 119.38) (end 144.145 118.11) (width 0.3) (layer F.Cu) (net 1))
 (segment (start 183.515 118.11) (end 183.515 114.3) (width 0.3) (layer F.Cu) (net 11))
 (segment (start 156.845 118.11) (end 156.845 114.3) (width 0.3) (layer F.Cu) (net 4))
 (segment (start 147.955 113.665) (end 149.86 111.76) (width 0.3) (layer F.Cu) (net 39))
 (segment (start 149.86 111.76) (end 150.495 111.76) (width 0.3) (layer F.Cu) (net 39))
 (segment (start 154.305 113.03) (end 154.305 114.3) (width 0.3) (layer F.Cu) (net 39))
 (segment (start 153.035 111.76) (end 154.305 113.03) (width 0.3) (layer F.Cu) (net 39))
 (segment (start 149.86 111.76) (end 150.495 111.76) (width 0.3) (layer F.Cu) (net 39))
 (segment (start 150.495 111.76) (end 153.035 111.76) (width 0.3) (layer F.Cu) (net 39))
 (segment (start 148.59 113.03) (end 149.86 111.76) (width 0.3) (layer F.Cu) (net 39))
 (segment (start 151.765 118.11) (end 151.765 114.3) (width 0.3) (layer F.Cu) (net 3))
 (segment (start 165.735 118.11) (end 165.735 114.3) (width 0.3) (layer F.Cu) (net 6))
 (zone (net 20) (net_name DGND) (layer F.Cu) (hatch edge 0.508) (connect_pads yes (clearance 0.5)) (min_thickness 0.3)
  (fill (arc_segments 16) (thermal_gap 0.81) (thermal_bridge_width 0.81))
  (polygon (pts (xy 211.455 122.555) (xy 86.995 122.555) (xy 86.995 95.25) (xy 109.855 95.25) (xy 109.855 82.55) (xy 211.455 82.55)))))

